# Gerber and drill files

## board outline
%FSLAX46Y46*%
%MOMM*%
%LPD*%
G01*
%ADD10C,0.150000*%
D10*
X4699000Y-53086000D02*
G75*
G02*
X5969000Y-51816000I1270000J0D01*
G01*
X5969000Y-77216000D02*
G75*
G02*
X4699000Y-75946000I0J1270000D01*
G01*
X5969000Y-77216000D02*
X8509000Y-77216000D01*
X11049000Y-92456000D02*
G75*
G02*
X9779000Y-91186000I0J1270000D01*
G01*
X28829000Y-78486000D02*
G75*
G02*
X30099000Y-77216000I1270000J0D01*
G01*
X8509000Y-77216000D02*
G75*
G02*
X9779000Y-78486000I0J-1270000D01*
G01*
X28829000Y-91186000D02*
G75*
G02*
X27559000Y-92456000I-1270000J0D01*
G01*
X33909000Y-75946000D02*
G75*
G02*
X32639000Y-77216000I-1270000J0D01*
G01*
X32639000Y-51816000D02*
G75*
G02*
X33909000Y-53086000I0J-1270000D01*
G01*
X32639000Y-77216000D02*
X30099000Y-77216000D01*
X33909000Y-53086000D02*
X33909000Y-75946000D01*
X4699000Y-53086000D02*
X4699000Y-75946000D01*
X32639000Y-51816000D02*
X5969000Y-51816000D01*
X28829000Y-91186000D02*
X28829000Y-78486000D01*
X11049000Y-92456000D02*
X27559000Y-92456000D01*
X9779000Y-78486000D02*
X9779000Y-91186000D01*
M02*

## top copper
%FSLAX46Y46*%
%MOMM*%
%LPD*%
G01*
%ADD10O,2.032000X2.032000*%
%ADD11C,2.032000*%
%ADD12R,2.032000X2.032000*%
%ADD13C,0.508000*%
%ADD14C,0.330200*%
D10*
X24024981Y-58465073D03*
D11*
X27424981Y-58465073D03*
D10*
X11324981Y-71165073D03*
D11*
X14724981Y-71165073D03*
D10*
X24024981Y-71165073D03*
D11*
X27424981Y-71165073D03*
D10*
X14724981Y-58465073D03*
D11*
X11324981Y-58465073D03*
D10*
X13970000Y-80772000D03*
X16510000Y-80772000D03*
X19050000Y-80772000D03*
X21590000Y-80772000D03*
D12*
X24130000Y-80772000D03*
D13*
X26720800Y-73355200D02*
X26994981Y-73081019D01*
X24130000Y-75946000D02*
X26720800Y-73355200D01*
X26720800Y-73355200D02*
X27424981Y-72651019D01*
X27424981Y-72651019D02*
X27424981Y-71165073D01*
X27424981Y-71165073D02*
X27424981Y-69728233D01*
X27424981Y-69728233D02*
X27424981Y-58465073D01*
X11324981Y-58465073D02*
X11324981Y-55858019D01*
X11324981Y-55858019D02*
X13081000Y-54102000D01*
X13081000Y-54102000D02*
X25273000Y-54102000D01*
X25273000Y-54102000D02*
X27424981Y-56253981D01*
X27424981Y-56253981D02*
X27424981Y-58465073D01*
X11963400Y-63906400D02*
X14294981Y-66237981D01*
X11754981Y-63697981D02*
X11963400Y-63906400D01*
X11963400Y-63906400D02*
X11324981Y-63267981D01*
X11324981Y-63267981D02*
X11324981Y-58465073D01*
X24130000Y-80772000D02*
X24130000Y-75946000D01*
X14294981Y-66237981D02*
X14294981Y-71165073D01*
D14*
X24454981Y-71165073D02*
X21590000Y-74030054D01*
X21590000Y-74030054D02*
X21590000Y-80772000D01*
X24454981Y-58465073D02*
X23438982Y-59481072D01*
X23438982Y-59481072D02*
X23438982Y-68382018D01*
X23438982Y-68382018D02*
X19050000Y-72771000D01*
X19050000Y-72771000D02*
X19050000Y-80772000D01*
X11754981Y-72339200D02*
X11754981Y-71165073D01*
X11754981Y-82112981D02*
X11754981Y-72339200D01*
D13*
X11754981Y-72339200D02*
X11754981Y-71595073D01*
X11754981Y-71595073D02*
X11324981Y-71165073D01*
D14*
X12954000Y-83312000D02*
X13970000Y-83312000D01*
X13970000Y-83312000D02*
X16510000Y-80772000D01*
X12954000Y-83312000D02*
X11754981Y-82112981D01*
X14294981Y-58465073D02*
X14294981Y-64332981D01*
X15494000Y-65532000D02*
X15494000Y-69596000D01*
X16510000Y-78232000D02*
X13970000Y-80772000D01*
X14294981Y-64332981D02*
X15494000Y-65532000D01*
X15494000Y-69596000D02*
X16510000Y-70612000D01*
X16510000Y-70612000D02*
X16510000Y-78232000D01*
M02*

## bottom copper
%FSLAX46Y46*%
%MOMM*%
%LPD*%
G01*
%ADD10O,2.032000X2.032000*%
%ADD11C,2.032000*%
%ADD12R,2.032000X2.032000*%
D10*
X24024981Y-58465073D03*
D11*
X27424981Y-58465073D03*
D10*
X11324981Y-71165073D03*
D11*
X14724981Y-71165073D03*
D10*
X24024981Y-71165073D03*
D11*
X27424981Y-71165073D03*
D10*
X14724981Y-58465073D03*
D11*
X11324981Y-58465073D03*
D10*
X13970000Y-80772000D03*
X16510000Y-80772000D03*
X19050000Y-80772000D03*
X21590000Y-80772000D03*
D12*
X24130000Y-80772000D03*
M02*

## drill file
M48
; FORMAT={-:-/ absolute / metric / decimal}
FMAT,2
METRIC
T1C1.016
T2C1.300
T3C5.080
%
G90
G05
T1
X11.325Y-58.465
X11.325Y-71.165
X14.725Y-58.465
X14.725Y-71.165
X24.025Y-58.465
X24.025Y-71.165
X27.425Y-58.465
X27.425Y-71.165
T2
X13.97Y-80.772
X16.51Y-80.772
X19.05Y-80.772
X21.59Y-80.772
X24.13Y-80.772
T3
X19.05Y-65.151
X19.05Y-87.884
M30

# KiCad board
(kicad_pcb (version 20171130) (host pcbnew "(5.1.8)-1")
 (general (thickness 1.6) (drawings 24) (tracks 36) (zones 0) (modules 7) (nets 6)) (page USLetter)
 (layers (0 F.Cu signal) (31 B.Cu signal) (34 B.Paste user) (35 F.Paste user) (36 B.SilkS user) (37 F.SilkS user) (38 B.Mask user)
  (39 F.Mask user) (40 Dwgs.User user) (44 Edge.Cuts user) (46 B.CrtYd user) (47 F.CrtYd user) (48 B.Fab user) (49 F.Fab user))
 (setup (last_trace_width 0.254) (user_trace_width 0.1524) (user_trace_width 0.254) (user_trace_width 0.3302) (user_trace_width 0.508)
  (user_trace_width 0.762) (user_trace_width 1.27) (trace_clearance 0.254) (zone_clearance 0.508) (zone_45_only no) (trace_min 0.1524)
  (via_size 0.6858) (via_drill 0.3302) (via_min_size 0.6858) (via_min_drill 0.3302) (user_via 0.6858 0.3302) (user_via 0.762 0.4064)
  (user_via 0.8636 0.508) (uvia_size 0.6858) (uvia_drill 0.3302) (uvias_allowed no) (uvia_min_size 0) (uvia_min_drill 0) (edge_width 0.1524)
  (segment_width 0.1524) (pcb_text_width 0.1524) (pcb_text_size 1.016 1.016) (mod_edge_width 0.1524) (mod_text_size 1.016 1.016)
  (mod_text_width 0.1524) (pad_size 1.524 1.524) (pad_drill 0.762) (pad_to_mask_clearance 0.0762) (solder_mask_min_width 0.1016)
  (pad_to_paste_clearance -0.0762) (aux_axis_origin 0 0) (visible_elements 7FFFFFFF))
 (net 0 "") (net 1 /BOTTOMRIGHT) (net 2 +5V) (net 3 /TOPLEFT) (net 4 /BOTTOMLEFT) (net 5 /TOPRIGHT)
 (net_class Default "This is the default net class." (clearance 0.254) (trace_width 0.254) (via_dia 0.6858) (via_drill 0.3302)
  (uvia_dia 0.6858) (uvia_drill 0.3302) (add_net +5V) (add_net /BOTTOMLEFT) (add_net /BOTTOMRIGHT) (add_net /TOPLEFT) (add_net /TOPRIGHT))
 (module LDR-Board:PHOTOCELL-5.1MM (layer F.Cu) (at 25.724981 58.465073 270)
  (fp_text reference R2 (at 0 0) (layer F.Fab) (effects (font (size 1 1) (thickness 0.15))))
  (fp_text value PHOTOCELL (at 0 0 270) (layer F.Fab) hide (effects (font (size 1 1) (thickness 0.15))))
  (pad 2 thru_hole oval (at 0 1.7 270) (size 2.032 2.032) (drill 1.016) (layers *.Cu *.Mask F.SilkS) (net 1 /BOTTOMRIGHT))
  (pad 1 thru_hole circle (at 0 -1.7 270) (size 2.032 2.032) (drill 1.016) (layers *.Cu *.Mask F.SilkS) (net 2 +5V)))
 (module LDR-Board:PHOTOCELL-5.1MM (layer F.Cu) (at 13.024981 71.165073 270)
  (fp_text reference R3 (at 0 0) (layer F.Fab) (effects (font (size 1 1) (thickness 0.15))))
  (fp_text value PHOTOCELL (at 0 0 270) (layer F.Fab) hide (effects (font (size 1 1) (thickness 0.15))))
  (pad 2 thru_hole oval (at 0 1.7 270) (size 2.032 2.032) (drill 1.016) (layers *.Cu *.Mask F.SilkS) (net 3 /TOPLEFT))
  (pad 1 thru_hole circle (at 0 -1.7 270) (size 2.032 2.032) (drill 1.016) (layers *.Cu *.Mask F.SilkS) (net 2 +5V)))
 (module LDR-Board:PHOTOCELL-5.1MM (layer F.Cu) (at 25.724981 71.165073 270)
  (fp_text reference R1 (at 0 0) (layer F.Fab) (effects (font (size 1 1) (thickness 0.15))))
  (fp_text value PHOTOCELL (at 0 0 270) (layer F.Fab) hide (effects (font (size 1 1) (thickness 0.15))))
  (pad 2 thru_hole oval (at 0 1.7 270) (size 2.032 2.032) (drill 1.016) (layers *.Cu *.Mask F.SilkS) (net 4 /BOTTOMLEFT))
  (pad 1 thru_hole circle (at 0 -1.7 270) (size 2.032 2.032) (drill 1.016) (layers *.Cu *.Mask F.SilkS) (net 2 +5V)))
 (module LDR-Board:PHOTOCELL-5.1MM (layer F.Cu) (at 13.024981 58.465073 90)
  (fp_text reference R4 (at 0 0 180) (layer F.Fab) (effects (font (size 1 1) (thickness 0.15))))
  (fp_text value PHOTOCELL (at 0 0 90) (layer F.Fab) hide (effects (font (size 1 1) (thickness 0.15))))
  (pad 2 thru_hole oval (at 0 1.7 90) (size 2.032 2.032) (drill 1.016) (layers *.Cu *.Mask F.SilkS) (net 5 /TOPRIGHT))
  (pad 1 thru_hole circle (at 0 -1.7 90) (size 2.032 2.032) (drill 1.016) (layers *.Cu *.Mask F.SilkS) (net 2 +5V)))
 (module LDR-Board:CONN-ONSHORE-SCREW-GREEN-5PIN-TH (layer F.Cu) (at 24.13 80.772 270)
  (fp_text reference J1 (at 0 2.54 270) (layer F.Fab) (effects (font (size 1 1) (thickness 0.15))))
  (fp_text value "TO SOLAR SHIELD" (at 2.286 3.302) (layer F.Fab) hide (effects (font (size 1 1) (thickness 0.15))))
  (pad 5 thru_hole oval (at 0 10.16 270) (size 2.032 2.032) (drill 1.3) (layers *.Cu *.Mask F.SilkS) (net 5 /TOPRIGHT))
  (pad 4 thru_hole oval (at 0 7.62 270) (size 2.032 2.032) (drill 1.3) (layers *.Cu *.Mask F.SilkS) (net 3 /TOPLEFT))
  (pad 3 thru_hole oval (at 0 5.08 270) (size 2.032 2.032) (drill 1.3) (layers *.Cu *.Mask F.SilkS) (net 1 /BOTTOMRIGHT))
  (pad 2 thru_hole oval (at 0 2.54 270) (size 2.032 2.032) (drill 1.3) (layers *.Cu *.Mask F.SilkS) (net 4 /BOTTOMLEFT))
  (pad 1 thru_hole rect (at 0 0 270) (size 2.032 2.032) (drill 1.3) (layers *.Cu *.Mask F.SilkS) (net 2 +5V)))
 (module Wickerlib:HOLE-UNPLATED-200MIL (layer F.Cu) (at 19.05 87.884)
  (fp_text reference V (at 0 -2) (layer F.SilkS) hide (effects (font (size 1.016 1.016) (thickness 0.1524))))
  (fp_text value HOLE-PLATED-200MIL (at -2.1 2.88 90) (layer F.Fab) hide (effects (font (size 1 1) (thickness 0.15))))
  (pad "" np_thru_hole circle (at 0 0) (size 5.08 5.08) (drill 5.08) (layers *.Cu)))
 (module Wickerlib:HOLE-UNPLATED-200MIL (layer F.Cu) (at 19.05 65.151)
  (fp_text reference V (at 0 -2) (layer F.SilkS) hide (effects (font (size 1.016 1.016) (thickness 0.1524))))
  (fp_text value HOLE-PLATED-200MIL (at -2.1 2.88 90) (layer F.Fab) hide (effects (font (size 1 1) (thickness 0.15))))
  (pad "" np_thru_hole circle (at 0 0) (size 5.08 5.08) (drill 5.08) (layers *.Cu)))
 (gr_arc (start 5.969 53.086) (end 4.699 53.086) (angle 90) (layer Edge.Cuts) (width 0.15))
 (gr_arc (start 5.969 75.946) (end 5.969 77.216) (angle 90) (layer Edge.Cuts) (width 0.15))
 (gr_line (start 5.969 77.216) (end 8.509 77.216) (layer Edge.Cuts) (width 0.15))
 (gr_arc (start 11.049 91.186) (end 11.049 92.456) (angle 90) (layer Edge.Cuts) (width 0.15))
 (gr_arc (start 30.099 78.486) (end 28.829 78.486) (angle 90) (layer Edge.Cuts) (width 0.15))
 (gr_arc (start 8.509 78.486) (end 8.509 77.216) (angle 90) (layer Edge.Cuts) (width 0.15))
 (gr_arc (start 27.559 91.186) (end 28.829 91.186) (angle 90) (layer Edge.Cuts) (width 0.15))
 (gr_arc (start 32.639 75.946) (end 33.909 75.946) (angle 90) (layer Edge.Cuts) (width 0.15))
 (gr_arc (start 32.639 53.086) (end 32.639 51.816) (angle 90) (layer Edge.Cuts) (width 0.15))
 (gr_line (start 32.639 77.216) (end 30.099 77.216) (layer Edge.Cuts) (width 0.15))
 (gr_line (start 33.909 53.086) (end 33.909 75.946) (layer Edge.Cuts) (width 0.15))
 (gr_line (start 4.699 53.086) (end 4.699 75.946) (layer Edge.Cuts) (width 0.15))
 (gr_line (start 32.639 51.816) (end 5.969 51.816) (layer Edge.Cuts) (width 0.15))
 (gr_line (start 28.829 91.186) (end 28.829 78.486) (layer Edge.Cuts) (width 0.15))
 (gr_line (start 11.049 92.456) (end 27.559 92.456) (layer Edge.Cuts) (width 0.15))
 (gr_line (start 9.779 78.486) (end 9.779 91.186) (layer Edge.Cuts) (width 0.15))
 (segment (start 26.7208 73.3552) (end 26.994981 73.081019) (width 0.508) (layer F.Cu) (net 2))
 (segment (start 24.13 75.946) (end 26.7208 73.3552) (width 0.508) (layer F.Cu) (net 2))
 (segment (start 26.7208 73.3552) (end 27.424981 72.651019) (width 0.508) (layer F.Cu) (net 2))
 (segment (start 27.424981 72.651019) (end 27.424981 71.165073) (width 0.508) (layer F.Cu) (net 2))
 (segment (start 27.424981 71.165073) (end 27.424981 69.728233) (width 0.508) (layer F.Cu) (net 2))
 (segment (start 27.424981 69.728233) (end 27.424981 58.465073) (width 0.508) (layer F.Cu) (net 2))
 (segment (start 11.324981 58.465073) (end 11.324981 55.858019) (width 0.508) (layer F.Cu) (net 2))
 (segment (start 11.324981 55.858019) (end 13.081 54.102) (width 0.508) (layer F.Cu) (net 2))
 (segment (start 13.081 54.102) (end 25.273 54.102) (width 0.508) (layer F.Cu) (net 2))
 (segment (start 25.273 54.102) (end 27.424981 56.253981) (width 0.508) (layer F.Cu) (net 2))
 (segment (start 27.424981 56.253981) (end 27.424981 58.465073) (width 0.508) (layer F.Cu) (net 2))
 (segment (start 11.9634 63.9064) (end 14.294981 66.237981) (width 0.508) (layer F.Cu) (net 2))
 (segment (start 11.754981 63.697981) (end 11.9634 63.9064) (width 0.508) (layer F.Cu) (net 2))
 (segment (start 11.9634 63.9064) (end 11.324981 63.267981) (width 0.508) (layer F.Cu) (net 2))
 (segment (start 11.324981 63.267981) (end 11.324981 58.465073) (width 0.508) (layer F.Cu) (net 2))
 (segment (start 24.13 80.772) (end 24.13 75.946) (width 0.508) (layer F.Cu) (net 2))
 (segment (start 14.294981 66.237981) (end 14.294981 71.165073) (width 0.508) (layer F.Cu) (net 2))
 (segment (start 24.454981 71.165073) (end 21.59 74.030054) (width 0.3302) (layer F.Cu) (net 4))
 (segment (start 21.59 74.030054) (end 21.59 80.772) (width 0.3302) (layer F.Cu) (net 4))
 (segment (start 24.454981 58.465073) (end 23.438982 59.481072) (width 0.3302) (layer F.Cu) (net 1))
 (segment (start 23.438982 59.481072) (end 23.438982 68.382018) (width 0.3302) (layer F.Cu) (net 1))
 (segment (start 23.438982 68.382018) (end 19.05 72.771) (width 0.3302) (layer F.Cu) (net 1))
 (segment (start 19.05 72.771) (end 19.05 80.772) (width 0.3302) (layer F.Cu) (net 1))
 (segment (start 11.754981 72.3392) (end 11.754981 71.165073) (width 0.3302) (layer F.Cu) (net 3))
 (segment (start 11.754981 82.112981) (end 11.754981 72.3392) (width 0.3302) (layer F.Cu) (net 3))
 (segment (start 11.754981 72.3392) (end 11.754981 71.595073) (width 0.508) (layer F.Cu) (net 3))
 (segment (start 11.754981 71.595073) (end 11.324981 71.165073) (width 0.508) (layer F.Cu) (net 3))
 (segment (start 12.954 83.312) (end 13.97 83.312) (width 0.3302) (layer F.Cu) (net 3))
 (segment (start 13.97 83.312) (end 16.51 80.772) (width 0.3302) (layer F.Cu) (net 3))
 (segment (start 12.954 83.312) (end 11.754981 82.112981) (width 0.3302) (layer F.Cu) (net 3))
 (segment (start 14.294981 58.465073) (end 14.294981 64.332981) (width 0.3302) (layer F.Cu) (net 5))
 (segment (start 15.494 65.532) (end 15.494 69.596) (width 0.3302) (layer F.Cu) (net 5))
 (segment (start 16.51 78.232) (end 13.97 80.772) (width 0.3302) (layer F.Cu) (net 5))
 (segment (start 14.294981 64.332981) (end 15.494 65.532) (width 0.3302) (layer F.Cu) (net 5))
 (segment (start 15.494 69.596) (end 16.51 70.612) (width 0.3302) (layer F.Cu) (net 5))
 (segment (start 16.51 70.612) (end 16.51 78.232) (width 0.3302) (layer F.Cu) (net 5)))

